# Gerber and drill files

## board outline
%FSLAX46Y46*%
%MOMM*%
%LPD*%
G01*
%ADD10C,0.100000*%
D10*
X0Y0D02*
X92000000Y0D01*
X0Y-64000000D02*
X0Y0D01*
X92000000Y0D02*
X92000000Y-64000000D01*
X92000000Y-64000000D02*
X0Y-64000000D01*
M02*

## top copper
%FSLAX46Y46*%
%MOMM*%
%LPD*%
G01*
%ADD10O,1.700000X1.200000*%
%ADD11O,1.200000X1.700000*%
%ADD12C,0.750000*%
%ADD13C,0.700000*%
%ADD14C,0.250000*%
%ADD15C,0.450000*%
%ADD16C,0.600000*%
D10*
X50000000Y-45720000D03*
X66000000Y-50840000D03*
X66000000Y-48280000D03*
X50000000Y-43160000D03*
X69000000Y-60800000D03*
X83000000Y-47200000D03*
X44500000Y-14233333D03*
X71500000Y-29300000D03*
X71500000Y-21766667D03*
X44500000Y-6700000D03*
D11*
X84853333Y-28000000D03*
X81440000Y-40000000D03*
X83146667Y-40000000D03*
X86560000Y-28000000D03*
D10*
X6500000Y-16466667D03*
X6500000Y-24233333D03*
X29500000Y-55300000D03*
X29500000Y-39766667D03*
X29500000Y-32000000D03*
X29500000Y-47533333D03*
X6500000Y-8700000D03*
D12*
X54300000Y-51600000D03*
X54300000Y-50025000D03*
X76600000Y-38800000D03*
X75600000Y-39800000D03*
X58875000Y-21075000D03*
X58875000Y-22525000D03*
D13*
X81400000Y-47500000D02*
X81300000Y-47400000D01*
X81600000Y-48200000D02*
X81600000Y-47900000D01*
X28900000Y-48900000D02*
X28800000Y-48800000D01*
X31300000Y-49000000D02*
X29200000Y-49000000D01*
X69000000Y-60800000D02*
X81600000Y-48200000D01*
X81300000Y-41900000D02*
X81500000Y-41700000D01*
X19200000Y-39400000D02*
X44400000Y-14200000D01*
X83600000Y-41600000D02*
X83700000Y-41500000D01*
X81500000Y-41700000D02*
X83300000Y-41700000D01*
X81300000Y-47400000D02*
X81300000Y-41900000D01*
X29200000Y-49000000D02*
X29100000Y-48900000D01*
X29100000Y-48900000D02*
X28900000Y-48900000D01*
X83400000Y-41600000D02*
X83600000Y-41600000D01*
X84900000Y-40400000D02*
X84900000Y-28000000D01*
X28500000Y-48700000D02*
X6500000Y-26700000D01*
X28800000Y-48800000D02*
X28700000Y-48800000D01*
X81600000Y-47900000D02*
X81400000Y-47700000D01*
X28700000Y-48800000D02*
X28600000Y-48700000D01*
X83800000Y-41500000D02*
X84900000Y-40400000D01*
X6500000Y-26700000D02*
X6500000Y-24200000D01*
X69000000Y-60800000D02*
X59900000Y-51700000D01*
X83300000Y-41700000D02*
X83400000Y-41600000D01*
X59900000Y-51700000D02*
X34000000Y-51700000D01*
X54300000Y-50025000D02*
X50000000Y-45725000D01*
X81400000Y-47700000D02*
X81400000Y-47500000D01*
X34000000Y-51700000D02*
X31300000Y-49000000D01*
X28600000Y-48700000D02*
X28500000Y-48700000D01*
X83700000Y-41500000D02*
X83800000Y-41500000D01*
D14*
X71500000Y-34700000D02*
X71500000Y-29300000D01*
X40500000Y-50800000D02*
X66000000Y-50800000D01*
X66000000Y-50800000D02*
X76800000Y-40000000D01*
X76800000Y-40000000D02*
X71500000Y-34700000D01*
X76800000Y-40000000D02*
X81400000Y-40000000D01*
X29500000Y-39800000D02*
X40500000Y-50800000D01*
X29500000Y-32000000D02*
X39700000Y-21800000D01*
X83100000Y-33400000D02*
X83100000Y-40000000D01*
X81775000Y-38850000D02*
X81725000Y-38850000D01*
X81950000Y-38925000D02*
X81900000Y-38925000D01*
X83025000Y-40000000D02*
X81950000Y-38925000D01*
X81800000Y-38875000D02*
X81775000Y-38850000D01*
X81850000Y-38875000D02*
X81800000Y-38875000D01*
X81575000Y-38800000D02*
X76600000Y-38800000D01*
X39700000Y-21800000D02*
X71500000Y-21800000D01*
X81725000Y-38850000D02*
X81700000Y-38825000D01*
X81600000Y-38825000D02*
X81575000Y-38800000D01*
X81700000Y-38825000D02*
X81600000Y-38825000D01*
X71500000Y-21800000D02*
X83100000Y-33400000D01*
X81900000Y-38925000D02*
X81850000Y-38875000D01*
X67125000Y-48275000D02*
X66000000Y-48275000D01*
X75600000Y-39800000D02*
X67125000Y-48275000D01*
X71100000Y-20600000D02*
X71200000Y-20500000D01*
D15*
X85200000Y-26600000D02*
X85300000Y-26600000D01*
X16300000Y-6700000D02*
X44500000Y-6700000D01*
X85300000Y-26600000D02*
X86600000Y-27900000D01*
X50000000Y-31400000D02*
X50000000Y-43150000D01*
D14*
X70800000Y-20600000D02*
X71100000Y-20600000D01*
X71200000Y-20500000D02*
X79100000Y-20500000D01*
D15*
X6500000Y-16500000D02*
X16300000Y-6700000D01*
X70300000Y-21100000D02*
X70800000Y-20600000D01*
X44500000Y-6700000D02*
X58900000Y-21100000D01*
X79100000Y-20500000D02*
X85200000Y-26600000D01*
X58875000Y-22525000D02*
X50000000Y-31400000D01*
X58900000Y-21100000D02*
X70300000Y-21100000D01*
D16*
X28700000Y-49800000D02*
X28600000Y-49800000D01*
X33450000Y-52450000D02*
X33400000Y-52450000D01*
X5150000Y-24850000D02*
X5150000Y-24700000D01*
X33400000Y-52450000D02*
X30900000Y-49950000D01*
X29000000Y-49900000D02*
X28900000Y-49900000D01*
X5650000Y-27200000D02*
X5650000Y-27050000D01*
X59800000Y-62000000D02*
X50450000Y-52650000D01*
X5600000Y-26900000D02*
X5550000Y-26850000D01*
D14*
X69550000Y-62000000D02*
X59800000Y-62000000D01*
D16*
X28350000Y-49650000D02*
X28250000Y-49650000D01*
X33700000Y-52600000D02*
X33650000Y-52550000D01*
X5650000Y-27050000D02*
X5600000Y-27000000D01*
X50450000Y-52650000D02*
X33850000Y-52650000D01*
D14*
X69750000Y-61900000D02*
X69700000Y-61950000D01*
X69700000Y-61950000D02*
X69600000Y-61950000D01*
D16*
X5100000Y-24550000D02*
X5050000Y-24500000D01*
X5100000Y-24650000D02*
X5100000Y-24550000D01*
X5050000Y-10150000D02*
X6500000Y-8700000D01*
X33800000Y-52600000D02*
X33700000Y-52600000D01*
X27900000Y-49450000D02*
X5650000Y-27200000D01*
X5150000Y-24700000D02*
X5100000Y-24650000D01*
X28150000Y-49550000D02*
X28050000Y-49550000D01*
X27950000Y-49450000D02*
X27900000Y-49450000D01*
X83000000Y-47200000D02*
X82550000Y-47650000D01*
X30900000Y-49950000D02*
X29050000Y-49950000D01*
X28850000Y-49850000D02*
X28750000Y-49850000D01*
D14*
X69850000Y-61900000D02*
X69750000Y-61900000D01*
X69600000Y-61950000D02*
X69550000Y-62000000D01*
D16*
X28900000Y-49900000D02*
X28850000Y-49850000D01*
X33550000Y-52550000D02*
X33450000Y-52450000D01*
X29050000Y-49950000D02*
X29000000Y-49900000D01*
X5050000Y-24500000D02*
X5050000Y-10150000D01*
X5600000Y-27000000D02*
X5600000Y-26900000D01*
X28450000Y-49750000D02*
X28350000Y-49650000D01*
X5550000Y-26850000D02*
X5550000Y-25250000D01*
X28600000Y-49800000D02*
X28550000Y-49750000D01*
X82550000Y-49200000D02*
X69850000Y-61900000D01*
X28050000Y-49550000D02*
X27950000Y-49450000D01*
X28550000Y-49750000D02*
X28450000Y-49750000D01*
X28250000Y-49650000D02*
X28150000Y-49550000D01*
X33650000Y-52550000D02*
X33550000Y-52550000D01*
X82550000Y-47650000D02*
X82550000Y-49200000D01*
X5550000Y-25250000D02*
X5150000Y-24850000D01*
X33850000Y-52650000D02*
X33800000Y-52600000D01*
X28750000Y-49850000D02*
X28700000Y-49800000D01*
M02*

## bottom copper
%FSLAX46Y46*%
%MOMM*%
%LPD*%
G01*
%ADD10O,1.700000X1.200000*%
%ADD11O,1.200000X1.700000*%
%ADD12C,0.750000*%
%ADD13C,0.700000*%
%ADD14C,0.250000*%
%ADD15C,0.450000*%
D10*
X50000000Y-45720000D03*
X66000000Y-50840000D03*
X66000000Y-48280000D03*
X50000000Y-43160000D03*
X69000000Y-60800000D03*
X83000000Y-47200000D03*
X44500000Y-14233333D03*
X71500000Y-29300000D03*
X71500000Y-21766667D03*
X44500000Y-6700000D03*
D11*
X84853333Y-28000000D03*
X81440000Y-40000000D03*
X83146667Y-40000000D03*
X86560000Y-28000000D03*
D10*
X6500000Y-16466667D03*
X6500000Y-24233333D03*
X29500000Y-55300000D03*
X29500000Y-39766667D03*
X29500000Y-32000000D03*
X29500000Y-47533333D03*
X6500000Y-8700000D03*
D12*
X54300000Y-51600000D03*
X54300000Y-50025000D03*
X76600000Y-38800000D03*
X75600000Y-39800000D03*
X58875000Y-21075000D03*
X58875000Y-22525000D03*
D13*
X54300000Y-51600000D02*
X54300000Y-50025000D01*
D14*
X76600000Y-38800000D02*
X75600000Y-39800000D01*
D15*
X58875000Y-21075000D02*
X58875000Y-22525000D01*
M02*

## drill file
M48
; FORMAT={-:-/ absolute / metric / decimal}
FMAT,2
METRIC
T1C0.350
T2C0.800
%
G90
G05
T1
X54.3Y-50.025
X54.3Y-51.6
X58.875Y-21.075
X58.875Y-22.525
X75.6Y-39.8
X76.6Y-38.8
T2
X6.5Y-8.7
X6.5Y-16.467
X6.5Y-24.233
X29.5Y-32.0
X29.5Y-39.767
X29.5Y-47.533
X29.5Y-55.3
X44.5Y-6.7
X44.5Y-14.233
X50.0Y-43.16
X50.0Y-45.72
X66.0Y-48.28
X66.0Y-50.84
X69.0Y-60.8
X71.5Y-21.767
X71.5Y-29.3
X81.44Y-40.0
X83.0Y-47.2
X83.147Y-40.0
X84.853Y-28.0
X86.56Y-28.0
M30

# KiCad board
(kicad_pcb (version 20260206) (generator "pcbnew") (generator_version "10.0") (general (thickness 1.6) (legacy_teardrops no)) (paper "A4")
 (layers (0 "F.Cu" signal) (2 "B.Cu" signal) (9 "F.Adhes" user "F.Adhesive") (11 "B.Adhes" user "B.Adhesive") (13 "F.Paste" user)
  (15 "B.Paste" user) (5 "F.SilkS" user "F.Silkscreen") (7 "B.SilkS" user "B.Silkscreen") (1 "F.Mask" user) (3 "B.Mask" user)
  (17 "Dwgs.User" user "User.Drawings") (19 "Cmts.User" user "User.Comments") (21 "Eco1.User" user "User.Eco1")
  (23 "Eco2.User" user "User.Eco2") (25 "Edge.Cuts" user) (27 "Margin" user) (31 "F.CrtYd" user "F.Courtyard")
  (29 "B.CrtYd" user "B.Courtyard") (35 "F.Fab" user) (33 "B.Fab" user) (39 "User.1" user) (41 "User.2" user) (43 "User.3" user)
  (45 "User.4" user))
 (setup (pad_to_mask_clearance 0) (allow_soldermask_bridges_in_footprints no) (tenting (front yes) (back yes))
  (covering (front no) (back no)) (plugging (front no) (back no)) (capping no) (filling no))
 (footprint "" (layer "F.Cu") (at 58 47)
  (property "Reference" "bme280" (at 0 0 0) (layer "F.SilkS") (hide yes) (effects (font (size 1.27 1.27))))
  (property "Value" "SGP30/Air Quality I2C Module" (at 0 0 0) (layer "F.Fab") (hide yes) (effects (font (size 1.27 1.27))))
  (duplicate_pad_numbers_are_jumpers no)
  (pad "GND" thru_hole oval (at -8 -1.28) (size 1.7 1.2) (drill 0.8) (layers "*.Cu") (remove_unused_layers no) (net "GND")
   (thermal_bridge_angle 45))
  (pad "SCL" thru_hole oval (at 8 3.84) (size 1.7 1.2) (drill 0.8) (layers "*.Cu") (remove_unused_layers no) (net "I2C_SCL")
   (thermal_bridge_angle 45))
  (pad "SDA" thru_hole oval (at 8 1.28) (size 1.7 1.2) (drill 0.8) (layers "*.Cu") (remove_unused_layers no) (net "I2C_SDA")
   (thermal_bridge_angle 45))
  (pad "VCC" thru_hole oval (at -8 -3.84) (size 1.7 1.2) (drill 0.8) (layers "*.Cu") (remove_unused_layers no) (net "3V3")
   (thermal_bridge_angle 45)))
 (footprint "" (layer "F.Cu") (at 76 54)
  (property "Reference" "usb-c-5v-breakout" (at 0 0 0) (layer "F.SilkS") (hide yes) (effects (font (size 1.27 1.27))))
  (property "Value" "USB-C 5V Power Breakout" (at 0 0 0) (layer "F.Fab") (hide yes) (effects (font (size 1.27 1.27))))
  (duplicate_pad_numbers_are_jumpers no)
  (pad "GND" thru_hole oval (at -7 6.8) (size 1.7 1.2) (drill 0.8) (layers "*.Cu") (remove_unused_layers no) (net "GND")
   (thermal_bridge_angle 45))
  (pad "VBUS" thru_hole oval (at 7 -6.8) (size 1.7 1.2) (drill 0.8) (layers "*.Cu") (remove_unused_layers no) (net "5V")
   (thermal_bridge_angle 45)))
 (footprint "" (layer "F.Cu") (at 58 18)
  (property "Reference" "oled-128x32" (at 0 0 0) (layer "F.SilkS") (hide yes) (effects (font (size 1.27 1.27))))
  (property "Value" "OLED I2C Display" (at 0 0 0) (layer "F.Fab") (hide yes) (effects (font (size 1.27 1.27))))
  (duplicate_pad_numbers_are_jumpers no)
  (pad "GND" thru_hole oval (at -13.5 -3.766667) (size 1.7 1.2) (drill 0.8) (layers "*.Cu") (remove_unused_layers no) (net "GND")
   (thermal_bridge_angle 45))
  (pad "SCL" thru_hole oval (at 13.5 11.3) (size 1.7 1.2) (drill 0.8) (layers "*.Cu") (remove_unused_layers no) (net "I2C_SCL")
   (thermal_bridge_angle 45))
  (pad "SDA" thru_hole oval (at 13.5 3.766667) (size 1.7 1.2) (drill 0.8) (layers "*.Cu") (remove_unused_layers no) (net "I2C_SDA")
   (thermal_bridge_angle 45))
  (pad "VCC" thru_hole oval (at -13.5 -11.3) (size 1.7 1.2) (drill 0.8) (layers "*.Cu") (remove_unused_layers no) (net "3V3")
   (thermal_bridge_angle 45)))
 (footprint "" (layer "F.Cu") (at 84 34 90)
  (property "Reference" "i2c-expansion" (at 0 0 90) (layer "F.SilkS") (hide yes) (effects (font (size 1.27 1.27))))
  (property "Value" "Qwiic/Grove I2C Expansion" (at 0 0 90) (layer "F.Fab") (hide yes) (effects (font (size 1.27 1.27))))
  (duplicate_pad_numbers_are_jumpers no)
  (pad "GND" thru_hole oval (at 6 0.853333 90) (size 1.7 1.2) (drill 0.8) (layers "*.Cu") (remove_unused_layers no) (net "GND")
   (thermal_bridge_angle 45))
  (pad "SCL" thru_hole oval (at -6 -2.56 90) (size 1.7 1.2) (drill 0.8) (layers "*.Cu") (remove_unused_layers no) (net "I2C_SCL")
   (thermal_bridge_angle 45))
  (pad "SDA" thru_hole oval (at -6 -0.853333 90) (size 1.7 1.2) (drill 0.8) (layers "*.Cu") (remove_unused_layers no) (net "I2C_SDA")
   (thermal_bridge_angle 45))
  (pad "VCC" thru_hole oval (at 6 2.56 90) (size 1.7 1.2) (drill 0.8) (layers "*.Cu") (remove_unused_layers no) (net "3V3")
   (thermal_bridge_angle 45)))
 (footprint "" (layer "F.Cu") (at 18 32)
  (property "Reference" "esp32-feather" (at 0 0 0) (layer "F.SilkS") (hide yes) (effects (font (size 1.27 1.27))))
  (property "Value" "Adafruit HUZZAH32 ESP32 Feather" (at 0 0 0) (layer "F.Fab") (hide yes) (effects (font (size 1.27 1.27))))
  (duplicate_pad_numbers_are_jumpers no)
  (pad "3V3" thru_hole oval (at -11.5 -15.533333) (size 1.7 1.2) (drill 0.8) (layers "*.Cu") (remove_unused_layers no) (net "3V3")
   (thermal_bridge_angle 45))
  (pad "GND" thru_hole oval (at -11.5 -7.766667) (size 1.7 1.2) (drill 0.8) (layers "*.Cu") (remove_unused_layers no) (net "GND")
   (thermal_bridge_angle 45))
  (pad "RX" thru_hole oval (at 11.5 23.3) (size 1.7 1.2) (drill 0.8) (layers "*.Cu") (remove_unused_layers no) (thermal_bridge_angle 45))
  (pad "SCL" thru_hole oval (at 11.5 7.766667) (size 1.7 1.2) (drill 0.8) (layers "*.Cu") (remove_unused_layers no) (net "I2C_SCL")
   (thermal_bridge_angle 45))
  (pad "SDA" thru_hole oval (at 11.5 0) (size 1.7 1.2) (drill 0.8) (layers "*.Cu") (remove_unused_layers no) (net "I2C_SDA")
   (thermal_bridge_angle 45))
  (pad "TX" thru_hole oval (at 11.5 15.533333) (size 1.7 1.2) (drill 0.8) (layers "*.Cu") (remove_unused_layers no)
   (thermal_bridge_angle 45))
  (pad "VIN" thru_hole oval (at -11.5 -23.3) (size 1.7 1.2) (drill 0.8) (layers "*.Cu") (remove_unused_layers no) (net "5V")
   (thermal_bridge_angle 45)))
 (gr_line (start 0 0) (end 92 0) (stroke (width 0.1) (type default)) (layer "Edge.Cuts"))
 (gr_line (start 0 64) (end 0 0) (stroke (width 0.1) (type default)) (layer "Edge.Cuts"))
 (gr_line (start 92 0) (end 92 64) (stroke (width 0.1) (type default)) (layer "Edge.Cuts"))
 (gr_line (start 92 64) (end 0 64) (stroke (width 0.1) (type default)) (layer "Edge.Cuts"))
 (segment (start 81.4 47.5) (end 81.3 47.4) (width 0.7) (layer "F.Cu") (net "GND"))
 (segment (start 81.6 48.2) (end 81.6 47.9) (width 0.7) (layer "F.Cu") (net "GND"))
 (segment (start 28.9 48.9) (end 28.8 48.8) (width 0.7) (layer "F.Cu") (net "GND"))
 (segment (start 31.3 49) (end 29.2 49) (width 0.7) (layer "F.Cu") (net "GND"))
 (segment (start 69 60.8) (end 81.6 48.2) (width 0.7) (layer "F.Cu") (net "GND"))
 (segment (start 81.3 41.9) (end 81.5 41.7) (width 0.7) (layer "F.Cu") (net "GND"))
 (segment (start 19.2 39.4) (end 44.4 14.2) (width 0.7) (layer "F.Cu") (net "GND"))
 (segment (start 83.6 41.6) (end 83.7 41.5) (width 0.7) (layer "F.Cu") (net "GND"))
 (segment (start 81.5 41.7) (end 83.3 41.7) (width 0.7) (layer "F.Cu") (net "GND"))
 (segment (start 81.3 47.4) (end 81.3 41.9) (width 0.7) (layer "F.Cu") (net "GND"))
 (segment (start 29.2 49) (end 29.1 48.9) (width 0.7) (layer "F.Cu") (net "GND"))
 (segment (start 29.1 48.9) (end 28.9 48.9) (width 0.7) (layer "F.Cu") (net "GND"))
 (segment (start 83.4 41.6) (end 83.6 41.6) (width 0.7) (layer "F.Cu") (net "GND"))
 (segment (start 84.9 40.4) (end 84.9 28) (width 0.7) (layer "F.Cu") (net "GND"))
 (segment (start 28.5 48.7) (end 6.5 26.7) (width 0.7) (layer "F.Cu") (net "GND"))
 (segment (start 28.8 48.8) (end 28.7 48.8) (width 0.7) (layer "F.Cu") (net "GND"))
 (segment (start 81.6 47.9) (end 81.4 47.7) (width 0.7) (layer "F.Cu") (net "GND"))
 (segment (start 28.7 48.8) (end 28.6 48.7) (width 0.7) (layer "F.Cu") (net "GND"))
 (segment (start 83.8 41.5) (end 84.9 40.4) (width 0.7) (layer "F.Cu") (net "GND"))
 (segment (start 6.5 26.7) (end 6.5 24.2) (width 0.7) (layer "F.Cu") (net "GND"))
 (segment (start 69 60.8) (end 59.9 51.7) (width 0.7) (layer "F.Cu") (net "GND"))
 (segment (start 83.3 41.7) (end 83.4 41.6) (width 0.7) (layer "F.Cu") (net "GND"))
 (segment (start 59.9 51.7) (end 34 51.7) (width 0.7) (layer "F.Cu") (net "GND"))
 (segment (start 54.3 50.025) (end 50 45.725) (width 0.7) (layer "F.Cu") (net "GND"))
 (segment (start 81.4 47.7) (end 81.4 47.5) (width 0.7) (layer "F.Cu") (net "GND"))
 (segment (start 34 51.7) (end 31.3 49) (width 0.7) (layer "F.Cu") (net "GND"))
 (segment (start 28.6 48.7) (end 28.5 48.7) (width 0.7) (layer "F.Cu") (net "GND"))
 (segment (start 83.7 41.5) (end 83.8 41.5) (width 0.7) (layer "F.Cu") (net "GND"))
 (via (at 54.3 51.6) (size 0.75) (drill 0.35) (layers "F.Cu" "B.Cu") (tenting (front yes) (back yes)) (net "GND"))
 (via (at 54.3 50.025) (size 0.75) (drill 0.35) (layers "F.Cu" "B.Cu") (tenting (front yes) (back yes)) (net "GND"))
 (segment (start 54.3 51.6) (end 54.3 50.025) (width 0.7) (layer "B.Cu") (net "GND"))
 (segment (start 71.5 34.7) (end 71.5 29.3) (width 0.25) (layer "F.Cu") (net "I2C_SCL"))
 (segment (start 40.5 50.8) (end 66 50.8) (width 0.25) (layer "F.Cu") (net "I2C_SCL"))
 (segment (start 66 50.8) (end 76.8 40) (width 0.25) (layer "F.Cu") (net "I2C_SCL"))
 (segment (start 76.8 40) (end 71.5 34.7) (width 0.25) (layer "F.Cu") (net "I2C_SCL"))
 (segment (start 76.8 40) (end 81.4 40) (width 0.25) (layer "F.Cu") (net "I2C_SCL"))
 (segment (start 29.5 39.8) (end 40.5 50.8) (width 0.25) (layer "F.Cu") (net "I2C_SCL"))
 (segment (start 29.5 32) (end 39.7 21.8) (width 0.25) (layer "F.Cu") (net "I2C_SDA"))
 (segment (start 83.1 33.4) (end 83.1 40) (width 0.25) (layer "F.Cu") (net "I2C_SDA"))
 (segment (start 81.775 38.85) (end 81.725 38.85) (width 0.25) (layer "F.Cu") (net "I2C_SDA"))
 (segment (start 81.95 38.925) (end 81.9 38.925) (width 0.25) (layer "F.Cu") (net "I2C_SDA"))
 (segment (start 83.025 40) (end 81.95 38.925) (width 0.25) (layer "F.Cu") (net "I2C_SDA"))
 (segment (start 81.8 38.875) (end 81.775 38.85) (width 0.25) (layer "F.Cu") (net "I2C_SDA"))
 (segment (start 81.85 38.875) (end 81.8 38.875) (width 0.25) (layer "F.Cu") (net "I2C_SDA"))
 (segment (start 81.575 38.8) (end 76.6 38.8) (width 0.25) (layer "F.Cu") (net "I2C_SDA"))
 (segment (start 39.7 21.8) (end 71.5 21.8) (width 0.25) (layer "F.Cu") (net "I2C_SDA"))
 (segment (start 81.725 38.85) (end 81.7 38.825) (width 0.25) (layer "F.Cu") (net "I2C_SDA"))
 (segment (start 81.6 38.825) (end 81.575 38.8) (width 0.25) (layer "F.Cu") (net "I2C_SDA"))
 (segment (start 81.7 38.825) (end 81.6 38.825) (width 0.25) (layer "F.Cu") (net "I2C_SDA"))
 (segment (start 71.5 21.8) (end 83.1 33.4) (width 0.25) (layer "F.Cu") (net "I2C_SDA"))
 (segment (start 81.9 38.925) (end 81.85 38.875) (width 0.25) (layer "F.Cu") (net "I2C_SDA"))
 (segment (start 67.125 48.275) (end 66 48.275) (width 0.25) (layer "F.Cu") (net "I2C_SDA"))
 (segment (start 75.6 39.8) (end 67.125 48.275) (width 0.25) (layer "F.Cu") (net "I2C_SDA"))
 (via (at 76.6 38.8) (size 0.75) (drill 0.35) (layers "F.Cu" "B.Cu") (tenting (front yes) (back yes)) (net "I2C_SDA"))
 (via (at 75.6 39.8) (size 0.75) (drill 0.35) (layers "F.Cu" "B.Cu") (tenting (front yes) (back yes)) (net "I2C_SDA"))
 (segment (start 76.6 38.8) (end 75.6 39.8) (width 0.25) (layer "B.Cu") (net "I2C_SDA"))
 (segment (start 71.1 20.6) (end 71.2 20.5) (width 0.25) (layer "F.Cu") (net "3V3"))
 (segment (start 85.2 26.6) (end 85.3 26.6) (width 0.45) (layer "F.Cu") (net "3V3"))
 (segment (start 16.3 6.7) (end 44.5 6.7) (width 0.45) (layer "F.Cu") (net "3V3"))
 (segment (start 85.3 26.6) (end 86.6 27.9) (width 0.45) (layer "F.Cu") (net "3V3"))
 (segment (start 50 31.4) (end 50 43.15) (width 0.45) (layer "F.Cu") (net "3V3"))
 (segment (start 70.8 20.6) (end 71.1 20.6) (width 0.25) (layer "F.Cu") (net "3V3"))
 (segment (start 71.2 20.5) (end 79.1 20.5) (width 0.25) (layer "F.Cu") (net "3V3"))
 (segment (start 6.5 16.5) (end 16.3 6.7) (width 0.45) (layer "F.Cu") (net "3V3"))
 (segment (start 70.3 21.1) (end 70.8 20.6) (width 0.45) (layer "F.Cu") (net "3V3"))
 (segment (start 44.5 6.7) (end 58.9 21.1) (width 0.45) (layer "F.Cu") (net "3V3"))
 (segment (start 79.1 20.5) (end 85.2 26.6) (width 0.45) (layer "F.Cu") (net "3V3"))
 (segment (start 58.875 22.525) (end 50 31.4) (width 0.45) (layer "F.Cu") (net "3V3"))
 (segment (start 58.9 21.1) (end 70.3 21.1) (width 0.45) (layer "F.Cu") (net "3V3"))
 (via (at 58.875 21.075) (size 0.75) (drill 0.35) (layers "F.Cu" "B.Cu") (tenting (front yes) (back yes)) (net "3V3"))
 (via (at 58.875 22.525) (size 0.75) (drill 0.35) (layers "F.Cu" "B.Cu") (tenting (front yes) (back yes)) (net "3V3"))
 (segment (start 58.875 21.075) (end 58.875 22.525) (width 0.45) (layer "B.Cu") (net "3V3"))
 (segment (start 28.7 49.8) (end 28.6 49.8) (width 0.6) (layer "F.Cu") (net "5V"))
 (segment (start 33.45 52.45) (end 33.4 52.45) (width 0.6) (layer "F.Cu") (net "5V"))
 (segment (start 5.15 24.85) (end 5.15 24.7) (width 0.6) (layer "F.Cu") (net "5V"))
 (segment (start 33.4 52.45) (end 30.9 49.95) (width 0.6) (layer "F.Cu") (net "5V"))
 (segment (start 29 49.9) (end 28.9 49.9) (width 0.6) (layer "F.Cu") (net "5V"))
 (segment (start 5.65 27.2) (end 5.65 27.05) (width 0.6) (layer "F.Cu") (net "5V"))
 (segment (start 59.8 62) (end 50.45 52.65) (width 0.6) (layer "F.Cu") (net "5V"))
 (segment (start 5.6 26.9) (end 5.55 26.85) (width 0.6) (layer "F.Cu") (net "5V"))
 (segment (start 69.55 62) (end 59.8 62) (width 0.25) (layer "F.Cu") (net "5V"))
 (segment (start 28.35 49.65) (end 28.25 49.65) (width 0.6) (layer "F.Cu") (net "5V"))
 (segment (start 33.7 52.6) (end 33.65 52.55) (width 0.6) (layer "F.Cu") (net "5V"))
 (segment (start 5.65 27.05) (end 5.6 27) (width 0.6) (layer "F.Cu") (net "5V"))
 (segment (start 50.45 52.65) (end 33.85 52.65) (width 0.6) (layer "F.Cu") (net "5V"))
 (segment (start 69.75 61.9) (end 69.7 61.95) (width 0.25) (layer "F.Cu") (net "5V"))
 (segment (start 69.7 61.95) (end 69.6 61.95) (width 0.25) (layer "F.Cu") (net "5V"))
 (segment (start 5.1 24.55) (end 5.05 24.5) (width 0.6) (layer "F.Cu") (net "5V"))
 (segment (start 5.1 24.65) (end 5.1 24.55) (width 0.6) (layer "F.Cu") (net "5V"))
 (segment (start 5.05 10.15) (end 6.5 8.7) (width 0.6) (layer "F.Cu") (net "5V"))
 (segment (start 33.8 52.6) (end 33.7 52.6) (width 0.6) (layer "F.Cu") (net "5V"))
 (segment (start 27.9 49.45) (end 5.65 27.2) (width 0.6) (layer "F.Cu") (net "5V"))
 (segment (start 5.15 24.7) (end 5.1 24.65) (width 0.6) (layer "F.Cu") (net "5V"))
 (segment (start 28.15 49.55) (end 28.05 49.55) (width 0.6) (layer "F.Cu") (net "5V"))
 (segment (start 27.95 49.45) (end 27.9 49.45) (width 0.6) (layer "F.Cu") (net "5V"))
 (segment (start 83 47.2) (end 82.55 47.65) (width 0.6) (layer "F.Cu") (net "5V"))
 (segment (start 30.9 49.95) (end 29.05 49.95) (width 0.6) (layer "F.Cu") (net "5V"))
 (segment (start 28.85 49.85) (end 28.75 49.85) (width 0.6) (layer "F.Cu") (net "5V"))
 (segment (start 69.85 61.9) (end 69.75 61.9) (width 0.25) (layer "F.Cu") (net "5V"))
 (segment (start 69.6 61.95) (end 69.55 62) (width 0.25) (layer "F.Cu") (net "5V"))
 (segment (start 28.9 49.9) (end 28.85 49.85) (width 0.6) (layer "F.Cu") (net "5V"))
 (segment (start 33.55 52.55) (end 33.45 52.45) (width 0.6) (layer "F.Cu") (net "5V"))
 (segment (start 29.05 49.95) (end 29 49.9) (width 0.6) (layer "F.Cu") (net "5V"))
 (segment (start 5.05 24.5) (end 5.05 10.15) (width 0.6) (layer "F.Cu") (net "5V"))
 (segment (start 5.6 27) (end 5.6 26.9) (width 0.6) (layer "F.Cu") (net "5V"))
 (segment (start 28.45 49.75) (end 28.35 49.65) (width 0.6) (layer "F.Cu") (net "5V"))
 (segment (start 5.55 26.85) (end 5.55 25.25) (width 0.6) (layer "F.Cu") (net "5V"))
 (segment (start 28.6 49.8) (end 28.55 49.75) (width 0.6) (layer "F.Cu") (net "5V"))
 (segment (start 82.55 49.2) (end 69.85 61.9) (width 0.6) (layer "F.Cu") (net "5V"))
 (segment (start 28.05 49.55) (end 27.95 49.45) (width 0.6) (layer "F.Cu") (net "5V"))
 (segment (start 28.55 49.75) (end 28.45 49.75) (width 0.6) (layer "F.Cu") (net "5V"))
 (segment (start 28.25 49.65) (end 28.15 49.55) (width 0.6) (layer "F.Cu") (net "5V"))
 (segment (start 33.65 52.55) (end 33.55 52.55) (width 0.6) (layer "F.Cu") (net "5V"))
 (segment (start 82.55 47.65) (end 82.55 49.2) (width 0.6) (layer "F.Cu") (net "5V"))
 (segment (start 5.55 25.25) (end 5.15 24.85) (width 0.6) (layer "F.Cu") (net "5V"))
 (segment (start 33.85 52.65) (end 33.8 52.6) (width 0.6) (layer "F.Cu") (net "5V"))
 (segment (start 28.75 49.85) (end 28.7 49.8) (width 0.6) (layer "F.Cu") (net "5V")))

